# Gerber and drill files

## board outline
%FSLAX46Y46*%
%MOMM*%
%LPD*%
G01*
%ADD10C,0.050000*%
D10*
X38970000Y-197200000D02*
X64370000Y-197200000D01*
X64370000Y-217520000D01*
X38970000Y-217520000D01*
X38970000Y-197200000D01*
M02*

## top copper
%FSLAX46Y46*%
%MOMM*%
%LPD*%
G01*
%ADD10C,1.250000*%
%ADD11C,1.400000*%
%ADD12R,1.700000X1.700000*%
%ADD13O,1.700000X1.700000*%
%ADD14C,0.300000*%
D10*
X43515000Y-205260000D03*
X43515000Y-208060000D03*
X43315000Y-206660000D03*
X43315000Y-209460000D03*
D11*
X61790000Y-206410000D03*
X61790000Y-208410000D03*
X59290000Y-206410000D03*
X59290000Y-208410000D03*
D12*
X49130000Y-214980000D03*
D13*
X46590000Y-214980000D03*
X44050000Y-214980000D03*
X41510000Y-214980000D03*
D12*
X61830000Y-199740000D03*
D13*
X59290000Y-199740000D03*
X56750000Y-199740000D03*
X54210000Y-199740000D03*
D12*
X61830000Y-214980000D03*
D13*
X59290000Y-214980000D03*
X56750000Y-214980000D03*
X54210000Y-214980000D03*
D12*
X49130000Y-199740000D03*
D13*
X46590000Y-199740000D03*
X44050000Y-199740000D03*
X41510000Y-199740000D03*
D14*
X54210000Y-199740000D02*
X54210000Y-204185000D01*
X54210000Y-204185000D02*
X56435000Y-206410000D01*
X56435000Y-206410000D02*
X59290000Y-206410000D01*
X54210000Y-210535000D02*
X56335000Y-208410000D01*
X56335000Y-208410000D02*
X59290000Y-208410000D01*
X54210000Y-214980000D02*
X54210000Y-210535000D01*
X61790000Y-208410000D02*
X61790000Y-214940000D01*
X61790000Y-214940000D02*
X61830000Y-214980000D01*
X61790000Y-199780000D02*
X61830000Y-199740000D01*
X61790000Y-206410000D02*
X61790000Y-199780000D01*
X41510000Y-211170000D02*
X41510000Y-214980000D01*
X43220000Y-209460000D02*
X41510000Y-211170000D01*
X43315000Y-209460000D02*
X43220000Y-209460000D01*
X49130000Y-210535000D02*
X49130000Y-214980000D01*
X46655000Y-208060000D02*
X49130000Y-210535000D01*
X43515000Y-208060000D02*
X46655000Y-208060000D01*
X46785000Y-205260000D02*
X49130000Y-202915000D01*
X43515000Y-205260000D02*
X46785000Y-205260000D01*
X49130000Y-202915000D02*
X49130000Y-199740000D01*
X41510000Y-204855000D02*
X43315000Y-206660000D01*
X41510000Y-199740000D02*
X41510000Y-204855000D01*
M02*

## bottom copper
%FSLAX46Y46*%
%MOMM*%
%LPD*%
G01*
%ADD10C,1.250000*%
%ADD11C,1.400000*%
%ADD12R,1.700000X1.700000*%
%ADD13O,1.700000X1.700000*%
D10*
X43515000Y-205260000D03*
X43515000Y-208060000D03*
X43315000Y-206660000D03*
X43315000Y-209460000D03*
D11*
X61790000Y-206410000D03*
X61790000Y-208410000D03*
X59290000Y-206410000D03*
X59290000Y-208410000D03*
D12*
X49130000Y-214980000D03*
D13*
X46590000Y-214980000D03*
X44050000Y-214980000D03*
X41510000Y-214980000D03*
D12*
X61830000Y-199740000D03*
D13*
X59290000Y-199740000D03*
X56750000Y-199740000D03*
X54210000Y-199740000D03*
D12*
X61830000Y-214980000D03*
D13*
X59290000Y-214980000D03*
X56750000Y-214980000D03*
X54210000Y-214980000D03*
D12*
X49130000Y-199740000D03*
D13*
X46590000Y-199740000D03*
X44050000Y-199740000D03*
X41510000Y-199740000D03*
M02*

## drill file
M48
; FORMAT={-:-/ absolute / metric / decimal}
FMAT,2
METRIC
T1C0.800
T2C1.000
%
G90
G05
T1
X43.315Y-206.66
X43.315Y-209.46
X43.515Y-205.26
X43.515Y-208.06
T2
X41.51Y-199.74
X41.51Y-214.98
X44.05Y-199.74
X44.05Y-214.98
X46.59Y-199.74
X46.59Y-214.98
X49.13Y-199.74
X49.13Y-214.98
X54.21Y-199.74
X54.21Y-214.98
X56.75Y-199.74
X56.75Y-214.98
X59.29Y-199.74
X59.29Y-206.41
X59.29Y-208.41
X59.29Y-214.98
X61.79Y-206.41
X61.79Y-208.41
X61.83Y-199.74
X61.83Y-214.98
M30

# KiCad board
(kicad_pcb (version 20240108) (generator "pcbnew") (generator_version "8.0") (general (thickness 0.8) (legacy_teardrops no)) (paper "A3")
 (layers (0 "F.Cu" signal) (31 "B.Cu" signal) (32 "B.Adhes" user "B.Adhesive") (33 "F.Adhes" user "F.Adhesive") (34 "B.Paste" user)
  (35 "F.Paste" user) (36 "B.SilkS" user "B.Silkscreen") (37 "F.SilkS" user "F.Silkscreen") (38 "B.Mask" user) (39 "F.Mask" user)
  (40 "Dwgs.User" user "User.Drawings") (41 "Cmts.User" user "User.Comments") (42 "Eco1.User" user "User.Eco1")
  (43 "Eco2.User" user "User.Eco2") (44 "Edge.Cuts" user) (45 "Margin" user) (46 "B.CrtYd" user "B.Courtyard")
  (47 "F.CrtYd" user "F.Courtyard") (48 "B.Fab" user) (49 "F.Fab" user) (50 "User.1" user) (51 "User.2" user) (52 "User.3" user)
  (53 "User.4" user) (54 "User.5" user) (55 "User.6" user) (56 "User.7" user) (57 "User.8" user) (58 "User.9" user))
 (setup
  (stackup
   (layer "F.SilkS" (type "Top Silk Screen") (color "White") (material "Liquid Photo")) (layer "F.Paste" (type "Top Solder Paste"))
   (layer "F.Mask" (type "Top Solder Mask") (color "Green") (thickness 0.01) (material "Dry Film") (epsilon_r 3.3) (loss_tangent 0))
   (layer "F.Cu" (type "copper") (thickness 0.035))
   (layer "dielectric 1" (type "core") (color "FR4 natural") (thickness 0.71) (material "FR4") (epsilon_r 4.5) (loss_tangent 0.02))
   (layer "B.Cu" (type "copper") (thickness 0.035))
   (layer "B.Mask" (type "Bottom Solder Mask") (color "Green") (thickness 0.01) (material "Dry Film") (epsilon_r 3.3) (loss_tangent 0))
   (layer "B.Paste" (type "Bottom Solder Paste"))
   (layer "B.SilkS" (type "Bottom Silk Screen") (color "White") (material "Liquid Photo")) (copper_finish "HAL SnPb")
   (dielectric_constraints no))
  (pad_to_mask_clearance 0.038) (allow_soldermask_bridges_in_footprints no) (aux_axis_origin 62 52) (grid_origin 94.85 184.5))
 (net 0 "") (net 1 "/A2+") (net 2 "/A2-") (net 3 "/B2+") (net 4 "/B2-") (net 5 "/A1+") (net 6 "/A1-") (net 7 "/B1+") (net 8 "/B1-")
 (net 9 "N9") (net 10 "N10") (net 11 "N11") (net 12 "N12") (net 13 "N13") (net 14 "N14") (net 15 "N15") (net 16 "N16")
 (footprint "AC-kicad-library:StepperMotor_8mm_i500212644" (layer "F.Cu") (at 43.415 207.36 180)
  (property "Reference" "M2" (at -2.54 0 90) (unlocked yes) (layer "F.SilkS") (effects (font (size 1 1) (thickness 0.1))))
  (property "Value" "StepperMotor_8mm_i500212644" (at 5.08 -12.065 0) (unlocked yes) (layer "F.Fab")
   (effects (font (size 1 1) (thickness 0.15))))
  (pad "1" thru_hole circle (at -0.1 2.1 180) (size 1.25 1.25) (drill 0.8) (layers "*.Cu" "*.Mask") (remove_unused_layers no) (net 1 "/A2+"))
  (pad "2" thru_hole circle (at -0.1 -0.7 180) (size 1.25 1.25) (drill 0.8) (layers "*.Cu" "*.Mask") (remove_unused_layers no)
   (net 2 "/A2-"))
  (pad "3" thru_hole circle (at 0.1 0.7 180) (size 1.25 1.25) (drill 0.8) (layers "*.Cu" "*.Mask") (remove_unused_layers no) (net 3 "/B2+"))
  (pad "4" thru_hole circle (at 0.1 -2.1 180) (size 1.25 1.25) (drill 0.8) (layers "*.Cu" "*.Mask") (remove_unused_layers no) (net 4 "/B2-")))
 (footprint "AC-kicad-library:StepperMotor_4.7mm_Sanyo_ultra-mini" (layer "F.Cu") (at 60.54 207.41)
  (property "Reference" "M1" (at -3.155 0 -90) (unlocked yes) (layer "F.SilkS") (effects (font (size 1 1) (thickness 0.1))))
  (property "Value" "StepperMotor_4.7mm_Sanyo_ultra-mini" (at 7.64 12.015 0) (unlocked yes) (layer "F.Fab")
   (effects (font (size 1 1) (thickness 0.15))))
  (pad "1" thru_hole circle (at 1.25 -1) (size 1.4 1.4) (drill 1) (layers "*.Cu" "*.Mask") (remove_unused_layers no) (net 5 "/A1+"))
  (pad "2" thru_hole circle (at 1.25 1) (size 1.4 1.4) (drill 1) (layers "*.Cu" "*.Mask") (remove_unused_layers no) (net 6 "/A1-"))
  (pad "3" thru_hole circle (at -1.25 -1) (size 1.4 1.4) (drill 1) (layers "*.Cu" "*.Mask") (remove_unused_layers no) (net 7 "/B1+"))
  (pad "4" thru_hole circle (at -1.25 1) (size 1.4 1.4) (drill 1) (layers "*.Cu" "*.Mask") (remove_unused_layers no) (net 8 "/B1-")))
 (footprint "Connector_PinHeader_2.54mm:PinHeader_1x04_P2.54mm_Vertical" (layer "B.Cu") (at 49.13 214.98 90)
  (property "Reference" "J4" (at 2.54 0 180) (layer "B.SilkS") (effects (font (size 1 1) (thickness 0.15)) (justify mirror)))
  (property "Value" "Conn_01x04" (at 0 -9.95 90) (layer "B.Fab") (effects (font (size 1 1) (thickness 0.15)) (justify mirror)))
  (pad "1" thru_hole rect (at 0 0 90) (size 1.7 1.7) (drill 1) (layers "*.Cu" "*.Mask") (remove_unused_layers no) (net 2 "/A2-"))
  (pad "2" thru_hole oval (at 0 -2.54 90) (size 1.7 1.7) (drill 1) (layers "*.Cu" "*.Mask") (remove_unused_layers no) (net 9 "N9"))
  (pad "3" thru_hole oval (at 0 -5.08 90) (size 1.7 1.7) (drill 1) (layers "*.Cu" "*.Mask") (remove_unused_layers no) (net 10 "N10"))
  (pad "4" thru_hole oval (at 0 -7.62 90) (size 1.7 1.7) (drill 1) (layers "*.Cu" "*.Mask") (remove_unused_layers no) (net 4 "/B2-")))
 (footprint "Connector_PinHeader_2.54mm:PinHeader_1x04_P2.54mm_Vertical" (layer "B.Cu") (at 61.83 199.74 90)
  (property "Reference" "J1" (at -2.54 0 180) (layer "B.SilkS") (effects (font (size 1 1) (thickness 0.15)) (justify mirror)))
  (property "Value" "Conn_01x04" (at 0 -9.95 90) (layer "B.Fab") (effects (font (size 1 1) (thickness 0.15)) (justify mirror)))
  (pad "1" thru_hole rect (at 0 0 90) (size 1.7 1.7) (drill 1) (layers "*.Cu" "*.Mask") (remove_unused_layers no) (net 5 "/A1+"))
  (pad "2" thru_hole oval (at 0 -2.54 90) (size 1.7 1.7) (drill 1) (layers "*.Cu" "*.Mask") (remove_unused_layers no) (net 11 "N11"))
  (pad "3" thru_hole oval (at 0 -5.08 90) (size 1.7 1.7) (drill 1) (layers "*.Cu" "*.Mask") (remove_unused_layers no) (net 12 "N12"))
  (pad "4" thru_hole oval (at 0 -7.62 90) (size 1.7 1.7) (drill 1) (layers "*.Cu" "*.Mask") (remove_unused_layers no) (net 7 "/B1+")))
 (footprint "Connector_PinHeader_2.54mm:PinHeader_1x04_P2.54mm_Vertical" (layer "B.Cu") (at 61.83 214.98 90)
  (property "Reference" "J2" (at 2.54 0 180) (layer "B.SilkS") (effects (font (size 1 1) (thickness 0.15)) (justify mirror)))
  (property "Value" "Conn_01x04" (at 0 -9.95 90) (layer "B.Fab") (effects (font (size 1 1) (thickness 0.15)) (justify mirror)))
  (pad "1" thru_hole rect (at 0 0 90) (size 1.7 1.7) (drill 1) (layers "*.Cu" "*.Mask") (remove_unused_layers no) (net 6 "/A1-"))
  (pad "2" thru_hole oval (at 0 -2.54 90) (size 1.7 1.7) (drill 1) (layers "*.Cu" "*.Mask") (remove_unused_layers no) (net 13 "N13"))
  (pad "3" thru_hole oval (at 0 -5.08 90) (size 1.7 1.7) (drill 1) (layers "*.Cu" "*.Mask") (remove_unused_layers no) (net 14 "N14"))
  (pad "4" thru_hole oval (at 0 -7.62 90) (size 1.7 1.7) (drill 1) (layers "*.Cu" "*.Mask") (remove_unused_layers no) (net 8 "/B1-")))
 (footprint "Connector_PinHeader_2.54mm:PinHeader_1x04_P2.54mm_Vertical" (layer "B.Cu") (at 49.13 199.74 90)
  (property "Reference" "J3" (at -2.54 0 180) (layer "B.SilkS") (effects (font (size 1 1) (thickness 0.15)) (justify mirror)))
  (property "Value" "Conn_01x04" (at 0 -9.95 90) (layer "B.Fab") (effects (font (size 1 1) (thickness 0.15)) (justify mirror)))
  (pad "1" thru_hole rect (at 0 0 90) (size 1.7 1.7) (drill 1) (layers "*.Cu" "*.Mask") (remove_unused_layers no) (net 1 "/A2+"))
  (pad "2" thru_hole oval (at 0 -2.54 90) (size 1.7 1.7) (drill 1) (layers "*.Cu" "*.Mask") (remove_unused_layers no) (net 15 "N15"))
  (pad "3" thru_hole oval (at 0 -5.08 90) (size 1.7 1.7) (drill 1) (layers "*.Cu" "*.Mask") (remove_unused_layers no) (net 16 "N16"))
  (pad "4" thru_hole oval (at 0 -7.62 90) (size 1.7 1.7) (drill 1) (layers "*.Cu" "*.Mask") (remove_unused_layers no) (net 3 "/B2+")))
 (gr_rect (start 38.97 197.2) (end 64.37 217.52) (stroke (width 0.05) (type default)) (fill none) (layer "Edge.Cuts"))
 (segment (start 54.21 199.74) (end 54.21 204.185) (width 0.3) (layer "F.Cu") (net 7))
 (segment (start 54.21 204.185) (end 56.435 206.41) (width 0.3) (layer "F.Cu") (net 7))
 (segment (start 56.435 206.41) (end 59.29 206.41) (width 0.3) (layer "F.Cu") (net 7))
 (segment (start 54.21 210.535) (end 56.335 208.41) (width 0.3) (layer "F.Cu") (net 8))
 (segment (start 56.335 208.41) (end 59.29 208.41) (width 0.3) (layer "F.Cu") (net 8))
 (segment (start 54.21 214.98) (end 54.21 210.535) (width 0.3) (layer "F.Cu") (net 8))
 (segment (start 61.79 208.41) (end 61.79 214.94) (width 0.3) (layer "F.Cu") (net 6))
 (segment (start 61.79 214.94) (end 61.83 214.98) (width 0.3) (layer "F.Cu") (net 6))
 (segment (start 61.79 199.78) (end 61.83 199.74) (width 0.3) (layer "F.Cu") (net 5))
 (segment (start 61.79 206.41) (end 61.79 199.78) (width 0.3) (layer "F.Cu") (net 5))
 (segment (start 41.51 211.17) (end 41.51 214.98) (width 0.3) (layer "F.Cu") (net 4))
 (segment (start 43.22 209.46) (end 41.51 211.17) (width 0.3) (layer "F.Cu") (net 4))
 (segment (start 43.315 209.46) (end 43.22 209.46) (width 0.3) (layer "F.Cu") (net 4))
 (segment (start 49.13 210.535) (end 49.13 214.98) (width 0.3) (layer "F.Cu") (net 2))
 (segment (start 46.655 208.06) (end 49.13 210.535) (width 0.3) (layer "F.Cu") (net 2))
 (segment (start 43.515 208.06) (end 46.655 208.06) (width 0.3) (layer "F.Cu") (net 2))
 (segment (start 46.785 205.26) (end 49.13 202.915) (width 0.3) (layer "F.Cu") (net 1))
 (segment (start 43.515 205.26) (end 46.785 205.26) (width 0.3) (layer "F.Cu") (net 1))
 (segment (start 49.13 202.915) (end 49.13 199.74) (width 0.3) (layer "F.Cu") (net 1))
 (segment (start 41.51 204.855) (end 43.315 206.66) (width 0.3) (layer "F.Cu") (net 3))
 (segment (start 41.51 199.74) (end 41.51 204.855) (width 0.3) (layer "F.Cu") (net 3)))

